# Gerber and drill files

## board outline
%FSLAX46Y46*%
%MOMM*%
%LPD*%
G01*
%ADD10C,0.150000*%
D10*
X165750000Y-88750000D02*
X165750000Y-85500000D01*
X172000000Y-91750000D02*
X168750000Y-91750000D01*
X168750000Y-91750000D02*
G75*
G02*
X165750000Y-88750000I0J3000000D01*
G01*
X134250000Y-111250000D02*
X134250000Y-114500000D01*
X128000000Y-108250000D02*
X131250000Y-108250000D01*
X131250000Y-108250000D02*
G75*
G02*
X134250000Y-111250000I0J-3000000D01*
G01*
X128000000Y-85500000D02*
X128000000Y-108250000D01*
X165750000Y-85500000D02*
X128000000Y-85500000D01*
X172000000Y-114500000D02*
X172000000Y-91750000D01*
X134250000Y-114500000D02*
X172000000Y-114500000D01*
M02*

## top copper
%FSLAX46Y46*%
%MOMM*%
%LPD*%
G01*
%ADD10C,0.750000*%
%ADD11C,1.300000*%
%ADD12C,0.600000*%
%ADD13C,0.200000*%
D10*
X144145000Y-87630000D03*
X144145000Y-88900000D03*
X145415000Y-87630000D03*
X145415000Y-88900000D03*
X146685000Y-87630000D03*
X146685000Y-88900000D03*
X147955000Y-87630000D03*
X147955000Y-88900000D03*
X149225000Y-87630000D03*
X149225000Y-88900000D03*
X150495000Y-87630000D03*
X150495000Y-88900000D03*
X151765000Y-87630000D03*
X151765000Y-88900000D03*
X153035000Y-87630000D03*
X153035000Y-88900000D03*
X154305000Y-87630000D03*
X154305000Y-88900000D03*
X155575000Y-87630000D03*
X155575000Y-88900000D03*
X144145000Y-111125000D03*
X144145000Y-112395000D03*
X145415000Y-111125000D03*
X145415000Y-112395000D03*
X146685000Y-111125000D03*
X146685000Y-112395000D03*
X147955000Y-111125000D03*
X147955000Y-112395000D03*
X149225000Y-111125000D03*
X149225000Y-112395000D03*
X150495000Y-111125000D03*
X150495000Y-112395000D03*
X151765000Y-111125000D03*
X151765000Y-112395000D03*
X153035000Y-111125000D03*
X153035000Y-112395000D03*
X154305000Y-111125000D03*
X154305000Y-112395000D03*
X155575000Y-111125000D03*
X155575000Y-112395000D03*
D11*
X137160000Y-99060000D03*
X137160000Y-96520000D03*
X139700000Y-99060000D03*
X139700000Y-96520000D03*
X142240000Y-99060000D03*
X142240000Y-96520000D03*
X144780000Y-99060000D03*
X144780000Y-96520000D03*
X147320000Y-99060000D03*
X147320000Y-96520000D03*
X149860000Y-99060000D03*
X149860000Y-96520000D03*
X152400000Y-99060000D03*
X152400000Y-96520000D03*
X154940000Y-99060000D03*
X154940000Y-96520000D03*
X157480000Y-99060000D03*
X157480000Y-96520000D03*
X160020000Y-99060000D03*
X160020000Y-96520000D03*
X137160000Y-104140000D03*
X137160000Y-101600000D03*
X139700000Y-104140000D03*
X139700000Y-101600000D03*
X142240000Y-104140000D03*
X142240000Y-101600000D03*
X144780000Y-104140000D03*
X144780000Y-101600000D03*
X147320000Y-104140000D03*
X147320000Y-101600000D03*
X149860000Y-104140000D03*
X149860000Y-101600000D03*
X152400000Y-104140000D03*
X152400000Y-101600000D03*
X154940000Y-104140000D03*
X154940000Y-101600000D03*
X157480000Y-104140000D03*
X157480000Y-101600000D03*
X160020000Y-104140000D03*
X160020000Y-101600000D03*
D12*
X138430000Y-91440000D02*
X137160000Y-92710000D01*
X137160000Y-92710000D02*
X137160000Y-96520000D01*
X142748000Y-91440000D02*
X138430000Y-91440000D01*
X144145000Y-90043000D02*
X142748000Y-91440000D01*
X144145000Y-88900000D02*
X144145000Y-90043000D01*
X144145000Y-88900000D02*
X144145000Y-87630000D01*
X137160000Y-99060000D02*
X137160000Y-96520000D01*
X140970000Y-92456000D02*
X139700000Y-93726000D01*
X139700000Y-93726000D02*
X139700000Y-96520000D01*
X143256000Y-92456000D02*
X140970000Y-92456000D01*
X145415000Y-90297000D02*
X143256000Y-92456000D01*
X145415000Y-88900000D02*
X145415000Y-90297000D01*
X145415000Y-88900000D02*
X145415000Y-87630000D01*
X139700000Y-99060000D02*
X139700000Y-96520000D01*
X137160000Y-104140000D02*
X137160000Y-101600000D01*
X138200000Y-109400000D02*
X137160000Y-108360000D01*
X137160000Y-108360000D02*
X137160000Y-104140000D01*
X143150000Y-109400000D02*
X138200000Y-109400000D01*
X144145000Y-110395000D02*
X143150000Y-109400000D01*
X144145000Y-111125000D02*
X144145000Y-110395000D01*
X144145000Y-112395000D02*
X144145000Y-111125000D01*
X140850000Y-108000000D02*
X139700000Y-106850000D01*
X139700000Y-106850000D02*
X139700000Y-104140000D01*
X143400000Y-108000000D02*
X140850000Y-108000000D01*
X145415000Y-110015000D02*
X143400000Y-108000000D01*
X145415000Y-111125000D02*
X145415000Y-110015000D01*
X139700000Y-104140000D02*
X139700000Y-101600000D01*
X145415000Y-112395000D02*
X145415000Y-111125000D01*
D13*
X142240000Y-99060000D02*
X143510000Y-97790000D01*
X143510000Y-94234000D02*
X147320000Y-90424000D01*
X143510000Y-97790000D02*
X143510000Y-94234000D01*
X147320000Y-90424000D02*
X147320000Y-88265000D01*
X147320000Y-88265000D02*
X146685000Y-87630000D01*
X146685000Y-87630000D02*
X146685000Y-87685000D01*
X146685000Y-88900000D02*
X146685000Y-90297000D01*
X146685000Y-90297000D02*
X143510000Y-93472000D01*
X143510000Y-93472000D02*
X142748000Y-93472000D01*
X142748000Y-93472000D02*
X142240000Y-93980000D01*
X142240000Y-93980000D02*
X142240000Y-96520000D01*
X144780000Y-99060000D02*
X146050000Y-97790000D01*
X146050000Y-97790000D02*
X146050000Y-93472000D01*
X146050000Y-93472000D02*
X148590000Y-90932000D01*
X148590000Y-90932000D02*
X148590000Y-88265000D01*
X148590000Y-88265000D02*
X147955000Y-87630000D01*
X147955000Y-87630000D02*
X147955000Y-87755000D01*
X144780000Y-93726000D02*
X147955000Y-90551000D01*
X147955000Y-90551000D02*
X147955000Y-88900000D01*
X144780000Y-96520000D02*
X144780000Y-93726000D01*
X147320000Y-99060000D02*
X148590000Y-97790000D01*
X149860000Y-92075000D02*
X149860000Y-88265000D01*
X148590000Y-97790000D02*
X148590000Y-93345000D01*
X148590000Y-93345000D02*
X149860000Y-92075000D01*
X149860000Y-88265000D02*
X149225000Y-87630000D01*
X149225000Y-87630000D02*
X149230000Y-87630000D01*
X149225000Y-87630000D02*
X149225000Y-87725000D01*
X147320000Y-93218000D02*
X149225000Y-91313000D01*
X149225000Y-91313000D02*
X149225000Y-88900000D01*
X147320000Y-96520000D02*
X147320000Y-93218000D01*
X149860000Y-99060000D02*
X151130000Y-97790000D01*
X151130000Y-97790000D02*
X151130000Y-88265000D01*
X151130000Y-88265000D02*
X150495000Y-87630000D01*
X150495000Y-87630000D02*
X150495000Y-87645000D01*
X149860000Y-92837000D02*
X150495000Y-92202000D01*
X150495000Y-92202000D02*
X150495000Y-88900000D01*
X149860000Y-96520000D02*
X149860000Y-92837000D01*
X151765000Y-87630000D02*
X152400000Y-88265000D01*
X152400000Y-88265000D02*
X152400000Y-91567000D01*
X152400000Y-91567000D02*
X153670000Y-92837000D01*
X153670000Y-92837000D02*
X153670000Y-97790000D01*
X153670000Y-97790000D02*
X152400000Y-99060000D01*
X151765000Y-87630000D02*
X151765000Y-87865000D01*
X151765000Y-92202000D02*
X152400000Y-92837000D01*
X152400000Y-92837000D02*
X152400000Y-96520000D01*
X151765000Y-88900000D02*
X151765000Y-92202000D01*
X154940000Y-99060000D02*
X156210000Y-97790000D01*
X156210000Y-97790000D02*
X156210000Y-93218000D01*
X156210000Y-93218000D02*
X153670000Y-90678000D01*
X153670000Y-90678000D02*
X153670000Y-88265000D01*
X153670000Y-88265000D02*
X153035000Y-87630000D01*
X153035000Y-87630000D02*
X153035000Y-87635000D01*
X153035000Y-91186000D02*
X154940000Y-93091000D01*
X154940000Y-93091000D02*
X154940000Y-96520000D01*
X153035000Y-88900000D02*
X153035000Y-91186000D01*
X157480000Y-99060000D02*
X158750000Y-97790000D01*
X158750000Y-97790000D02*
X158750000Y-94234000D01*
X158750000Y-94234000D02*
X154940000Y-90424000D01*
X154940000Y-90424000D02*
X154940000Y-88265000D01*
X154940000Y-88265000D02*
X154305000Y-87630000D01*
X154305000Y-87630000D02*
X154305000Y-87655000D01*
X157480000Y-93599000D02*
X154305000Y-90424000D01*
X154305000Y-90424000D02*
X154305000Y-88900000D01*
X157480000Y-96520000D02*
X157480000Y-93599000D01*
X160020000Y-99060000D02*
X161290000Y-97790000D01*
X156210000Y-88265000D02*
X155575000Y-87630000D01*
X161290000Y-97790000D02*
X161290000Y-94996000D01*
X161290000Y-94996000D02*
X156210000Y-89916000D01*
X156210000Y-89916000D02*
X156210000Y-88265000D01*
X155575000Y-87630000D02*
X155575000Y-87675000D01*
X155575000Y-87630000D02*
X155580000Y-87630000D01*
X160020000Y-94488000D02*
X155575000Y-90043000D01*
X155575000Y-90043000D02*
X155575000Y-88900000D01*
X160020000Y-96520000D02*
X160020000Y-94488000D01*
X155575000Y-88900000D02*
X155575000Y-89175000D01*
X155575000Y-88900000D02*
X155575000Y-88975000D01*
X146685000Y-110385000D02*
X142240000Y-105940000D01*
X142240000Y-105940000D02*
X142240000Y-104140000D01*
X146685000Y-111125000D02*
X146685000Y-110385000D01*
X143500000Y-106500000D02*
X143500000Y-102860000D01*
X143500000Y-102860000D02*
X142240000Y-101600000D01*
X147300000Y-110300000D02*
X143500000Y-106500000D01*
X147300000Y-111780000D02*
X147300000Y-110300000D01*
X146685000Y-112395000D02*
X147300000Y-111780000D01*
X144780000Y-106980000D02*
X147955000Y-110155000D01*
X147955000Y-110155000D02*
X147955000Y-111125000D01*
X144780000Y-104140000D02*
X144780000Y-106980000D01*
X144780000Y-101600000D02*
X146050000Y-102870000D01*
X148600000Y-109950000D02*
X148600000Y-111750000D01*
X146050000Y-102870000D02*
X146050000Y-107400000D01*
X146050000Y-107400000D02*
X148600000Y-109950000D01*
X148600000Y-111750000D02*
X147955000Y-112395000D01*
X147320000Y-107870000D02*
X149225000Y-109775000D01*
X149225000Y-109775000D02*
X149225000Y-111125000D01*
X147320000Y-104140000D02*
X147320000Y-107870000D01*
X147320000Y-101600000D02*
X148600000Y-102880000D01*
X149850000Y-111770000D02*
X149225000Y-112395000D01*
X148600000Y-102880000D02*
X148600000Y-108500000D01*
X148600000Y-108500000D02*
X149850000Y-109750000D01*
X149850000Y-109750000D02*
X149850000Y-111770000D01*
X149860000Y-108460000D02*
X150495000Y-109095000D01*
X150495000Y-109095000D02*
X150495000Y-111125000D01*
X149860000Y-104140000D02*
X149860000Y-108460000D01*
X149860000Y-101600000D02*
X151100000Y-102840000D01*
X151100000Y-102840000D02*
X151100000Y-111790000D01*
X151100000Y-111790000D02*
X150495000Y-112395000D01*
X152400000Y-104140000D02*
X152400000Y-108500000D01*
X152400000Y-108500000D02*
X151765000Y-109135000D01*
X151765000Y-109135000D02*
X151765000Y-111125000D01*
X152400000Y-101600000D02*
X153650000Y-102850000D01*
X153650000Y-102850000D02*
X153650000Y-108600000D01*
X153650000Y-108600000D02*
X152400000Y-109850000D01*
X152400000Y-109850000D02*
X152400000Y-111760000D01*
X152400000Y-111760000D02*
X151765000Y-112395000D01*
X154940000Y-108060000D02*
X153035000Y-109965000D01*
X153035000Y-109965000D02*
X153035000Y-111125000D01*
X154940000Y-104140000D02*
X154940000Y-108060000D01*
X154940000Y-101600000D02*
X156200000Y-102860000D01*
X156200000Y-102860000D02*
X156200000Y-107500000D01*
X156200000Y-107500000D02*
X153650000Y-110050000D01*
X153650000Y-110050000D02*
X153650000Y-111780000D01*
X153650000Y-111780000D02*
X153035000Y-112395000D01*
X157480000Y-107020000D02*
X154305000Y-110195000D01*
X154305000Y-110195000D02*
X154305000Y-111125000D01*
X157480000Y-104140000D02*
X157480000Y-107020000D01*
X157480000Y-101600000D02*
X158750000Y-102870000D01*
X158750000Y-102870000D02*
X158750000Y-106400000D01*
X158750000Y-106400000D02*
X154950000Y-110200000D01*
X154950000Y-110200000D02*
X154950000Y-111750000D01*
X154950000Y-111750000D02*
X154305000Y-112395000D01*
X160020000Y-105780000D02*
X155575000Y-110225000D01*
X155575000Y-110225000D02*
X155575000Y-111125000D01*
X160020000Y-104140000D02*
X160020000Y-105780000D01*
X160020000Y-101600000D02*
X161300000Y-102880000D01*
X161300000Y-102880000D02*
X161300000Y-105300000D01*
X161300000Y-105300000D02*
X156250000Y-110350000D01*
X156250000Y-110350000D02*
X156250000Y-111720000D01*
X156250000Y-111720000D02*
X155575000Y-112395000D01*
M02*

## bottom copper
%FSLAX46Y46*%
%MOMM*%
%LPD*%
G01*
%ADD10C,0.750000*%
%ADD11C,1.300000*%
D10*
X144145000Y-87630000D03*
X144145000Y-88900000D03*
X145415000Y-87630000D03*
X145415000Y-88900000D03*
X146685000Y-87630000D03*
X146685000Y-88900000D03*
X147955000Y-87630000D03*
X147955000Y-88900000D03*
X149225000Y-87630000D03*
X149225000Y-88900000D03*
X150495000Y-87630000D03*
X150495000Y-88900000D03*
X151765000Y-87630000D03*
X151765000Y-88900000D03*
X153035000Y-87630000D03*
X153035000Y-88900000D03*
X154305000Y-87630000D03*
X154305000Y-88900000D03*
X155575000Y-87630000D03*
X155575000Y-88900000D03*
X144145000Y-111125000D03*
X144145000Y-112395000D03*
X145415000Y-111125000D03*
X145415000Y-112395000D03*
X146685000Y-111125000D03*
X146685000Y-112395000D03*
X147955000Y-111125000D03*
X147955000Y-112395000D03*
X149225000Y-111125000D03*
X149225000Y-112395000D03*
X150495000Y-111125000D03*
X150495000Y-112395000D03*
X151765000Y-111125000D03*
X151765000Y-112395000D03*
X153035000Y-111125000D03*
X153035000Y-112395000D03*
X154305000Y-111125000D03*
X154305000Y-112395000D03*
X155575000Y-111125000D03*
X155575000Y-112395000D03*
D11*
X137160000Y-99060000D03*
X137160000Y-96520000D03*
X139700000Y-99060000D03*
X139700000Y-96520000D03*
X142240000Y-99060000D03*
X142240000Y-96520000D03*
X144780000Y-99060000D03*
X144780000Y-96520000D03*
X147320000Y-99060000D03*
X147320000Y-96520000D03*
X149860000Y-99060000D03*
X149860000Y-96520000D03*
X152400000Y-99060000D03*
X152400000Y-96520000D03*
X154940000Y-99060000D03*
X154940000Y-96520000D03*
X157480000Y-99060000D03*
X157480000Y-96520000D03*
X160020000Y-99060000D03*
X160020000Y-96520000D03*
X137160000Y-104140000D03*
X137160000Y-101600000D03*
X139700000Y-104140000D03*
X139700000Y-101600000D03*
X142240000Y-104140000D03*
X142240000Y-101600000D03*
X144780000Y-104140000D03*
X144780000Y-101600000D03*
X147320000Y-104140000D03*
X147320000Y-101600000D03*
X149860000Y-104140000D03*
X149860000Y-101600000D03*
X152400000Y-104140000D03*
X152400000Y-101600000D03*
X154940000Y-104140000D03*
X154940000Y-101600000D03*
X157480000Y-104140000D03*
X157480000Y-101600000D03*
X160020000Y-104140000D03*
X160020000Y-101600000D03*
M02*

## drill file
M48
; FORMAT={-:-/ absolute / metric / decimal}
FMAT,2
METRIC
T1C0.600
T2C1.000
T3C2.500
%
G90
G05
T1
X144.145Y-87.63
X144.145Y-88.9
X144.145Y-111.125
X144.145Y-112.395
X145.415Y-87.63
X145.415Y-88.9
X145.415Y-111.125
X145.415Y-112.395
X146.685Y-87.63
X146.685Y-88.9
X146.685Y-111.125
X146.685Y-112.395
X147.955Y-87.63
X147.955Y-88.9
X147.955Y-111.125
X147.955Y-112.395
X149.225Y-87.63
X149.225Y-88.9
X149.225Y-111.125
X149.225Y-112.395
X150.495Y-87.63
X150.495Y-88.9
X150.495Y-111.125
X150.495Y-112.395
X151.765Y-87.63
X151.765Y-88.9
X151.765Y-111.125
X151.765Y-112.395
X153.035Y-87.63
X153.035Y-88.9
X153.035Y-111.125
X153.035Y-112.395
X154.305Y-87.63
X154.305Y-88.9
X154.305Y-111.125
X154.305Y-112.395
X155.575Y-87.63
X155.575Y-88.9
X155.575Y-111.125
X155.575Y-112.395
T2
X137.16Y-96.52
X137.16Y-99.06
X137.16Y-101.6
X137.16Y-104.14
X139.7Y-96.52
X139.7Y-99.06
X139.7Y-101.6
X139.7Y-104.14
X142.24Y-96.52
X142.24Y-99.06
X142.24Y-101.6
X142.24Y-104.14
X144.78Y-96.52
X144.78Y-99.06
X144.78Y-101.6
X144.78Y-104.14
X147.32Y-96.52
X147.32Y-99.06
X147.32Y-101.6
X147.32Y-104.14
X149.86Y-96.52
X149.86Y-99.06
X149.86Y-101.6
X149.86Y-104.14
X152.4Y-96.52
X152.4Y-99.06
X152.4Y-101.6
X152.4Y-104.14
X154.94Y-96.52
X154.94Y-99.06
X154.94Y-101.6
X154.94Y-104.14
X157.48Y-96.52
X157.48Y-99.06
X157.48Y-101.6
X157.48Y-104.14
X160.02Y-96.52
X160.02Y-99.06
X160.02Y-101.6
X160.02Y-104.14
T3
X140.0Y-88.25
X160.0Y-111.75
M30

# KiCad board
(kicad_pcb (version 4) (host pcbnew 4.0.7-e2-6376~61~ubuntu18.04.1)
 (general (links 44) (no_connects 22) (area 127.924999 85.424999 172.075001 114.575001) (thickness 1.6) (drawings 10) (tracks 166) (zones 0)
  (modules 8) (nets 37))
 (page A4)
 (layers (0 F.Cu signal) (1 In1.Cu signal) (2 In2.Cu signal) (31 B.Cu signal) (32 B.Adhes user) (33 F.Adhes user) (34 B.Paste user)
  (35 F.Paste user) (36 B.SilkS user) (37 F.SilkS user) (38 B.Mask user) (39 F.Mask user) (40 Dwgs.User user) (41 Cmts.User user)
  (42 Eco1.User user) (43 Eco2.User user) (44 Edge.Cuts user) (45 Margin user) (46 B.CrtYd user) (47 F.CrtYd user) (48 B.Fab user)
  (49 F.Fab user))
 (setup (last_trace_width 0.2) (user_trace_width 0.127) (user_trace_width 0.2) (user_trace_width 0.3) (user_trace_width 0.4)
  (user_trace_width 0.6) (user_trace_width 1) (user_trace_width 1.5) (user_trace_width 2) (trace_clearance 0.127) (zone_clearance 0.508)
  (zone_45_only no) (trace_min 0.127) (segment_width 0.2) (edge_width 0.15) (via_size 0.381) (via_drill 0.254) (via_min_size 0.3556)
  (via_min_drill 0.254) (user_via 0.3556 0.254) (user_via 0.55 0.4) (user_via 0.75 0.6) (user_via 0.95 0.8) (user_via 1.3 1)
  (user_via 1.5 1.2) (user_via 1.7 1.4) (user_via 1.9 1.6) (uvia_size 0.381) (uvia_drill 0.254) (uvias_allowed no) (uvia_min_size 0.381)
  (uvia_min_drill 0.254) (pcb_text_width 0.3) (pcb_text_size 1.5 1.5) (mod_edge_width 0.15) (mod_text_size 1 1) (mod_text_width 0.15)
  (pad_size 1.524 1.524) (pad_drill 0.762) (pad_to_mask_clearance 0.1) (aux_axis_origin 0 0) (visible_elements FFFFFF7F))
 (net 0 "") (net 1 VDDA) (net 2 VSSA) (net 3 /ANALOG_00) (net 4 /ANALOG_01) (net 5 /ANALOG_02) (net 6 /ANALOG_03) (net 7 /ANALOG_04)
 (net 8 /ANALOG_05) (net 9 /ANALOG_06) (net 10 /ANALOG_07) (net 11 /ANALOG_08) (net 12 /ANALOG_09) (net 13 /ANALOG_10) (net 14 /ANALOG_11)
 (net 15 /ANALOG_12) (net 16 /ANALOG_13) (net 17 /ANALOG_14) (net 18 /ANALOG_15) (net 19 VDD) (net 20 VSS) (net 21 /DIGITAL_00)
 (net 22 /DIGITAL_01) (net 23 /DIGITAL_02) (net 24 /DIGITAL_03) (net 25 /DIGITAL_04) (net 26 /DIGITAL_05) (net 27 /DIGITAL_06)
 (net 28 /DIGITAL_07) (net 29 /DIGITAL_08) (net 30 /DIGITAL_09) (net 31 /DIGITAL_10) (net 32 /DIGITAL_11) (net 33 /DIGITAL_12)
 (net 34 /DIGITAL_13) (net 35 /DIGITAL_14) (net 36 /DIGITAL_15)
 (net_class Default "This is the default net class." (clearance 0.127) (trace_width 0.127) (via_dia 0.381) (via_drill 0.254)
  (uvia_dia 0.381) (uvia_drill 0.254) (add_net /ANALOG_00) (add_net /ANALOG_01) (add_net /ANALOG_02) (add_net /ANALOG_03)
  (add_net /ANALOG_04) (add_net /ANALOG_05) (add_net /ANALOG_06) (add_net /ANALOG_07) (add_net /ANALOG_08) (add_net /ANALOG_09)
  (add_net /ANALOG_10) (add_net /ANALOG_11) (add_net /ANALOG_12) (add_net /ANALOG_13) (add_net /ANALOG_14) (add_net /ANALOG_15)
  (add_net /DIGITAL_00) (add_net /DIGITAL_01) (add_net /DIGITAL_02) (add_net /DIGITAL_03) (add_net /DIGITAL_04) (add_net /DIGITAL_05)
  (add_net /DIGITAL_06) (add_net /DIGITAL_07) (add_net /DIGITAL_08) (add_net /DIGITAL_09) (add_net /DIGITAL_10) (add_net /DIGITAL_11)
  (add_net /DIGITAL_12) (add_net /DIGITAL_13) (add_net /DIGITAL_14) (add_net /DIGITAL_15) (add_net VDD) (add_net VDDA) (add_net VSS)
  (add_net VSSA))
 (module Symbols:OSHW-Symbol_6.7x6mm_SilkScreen (layer F.Cu) (at 165.735 100.33 90)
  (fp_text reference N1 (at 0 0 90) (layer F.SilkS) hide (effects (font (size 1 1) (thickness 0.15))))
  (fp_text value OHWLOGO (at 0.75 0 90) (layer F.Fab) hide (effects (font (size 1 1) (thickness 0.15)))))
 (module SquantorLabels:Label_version (layer F.Cu) (at 170 100 90)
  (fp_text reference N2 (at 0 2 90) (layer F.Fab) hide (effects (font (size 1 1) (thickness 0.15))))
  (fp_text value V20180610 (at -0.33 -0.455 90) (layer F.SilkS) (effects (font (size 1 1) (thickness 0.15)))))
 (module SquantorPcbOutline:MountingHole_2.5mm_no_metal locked (layer F.Cu) (at 140 88.25)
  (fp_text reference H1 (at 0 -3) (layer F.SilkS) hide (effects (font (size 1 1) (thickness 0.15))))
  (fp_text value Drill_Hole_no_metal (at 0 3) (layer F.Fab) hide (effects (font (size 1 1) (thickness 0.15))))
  (pad "" np_thru_hole circle (at 0 0) (size 2.5 2.5) (drill 2.5) (layers *.Cu *.Mask)))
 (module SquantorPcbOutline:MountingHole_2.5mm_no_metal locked (layer F.Cu) (at 160 111.75)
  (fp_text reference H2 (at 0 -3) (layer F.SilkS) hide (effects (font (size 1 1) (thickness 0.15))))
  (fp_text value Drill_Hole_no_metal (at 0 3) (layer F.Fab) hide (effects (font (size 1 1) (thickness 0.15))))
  (pad "" np_thru_hole circle (at 0 0) (size 2.5 2.5) (drill 2.5) (layers *.Cu *.Mask)))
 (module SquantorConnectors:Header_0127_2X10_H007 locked (layer F.Cu) (at 149.86 88.265)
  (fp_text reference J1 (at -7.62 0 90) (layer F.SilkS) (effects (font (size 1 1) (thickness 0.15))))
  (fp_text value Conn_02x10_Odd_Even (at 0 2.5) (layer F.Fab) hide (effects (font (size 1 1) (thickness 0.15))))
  (pad 1 thru_hole circle (at -5.715 -0.635) (size 0.75 0.75) (drill 0.6) (layers *.Cu *.Mask) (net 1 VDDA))
  (pad 2 thru_hole circle (at -5.715 0.635) (size 0.75 0.75) (drill 0.6) (layers *.Cu *.Mask) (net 1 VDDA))
  (pad 3 thru_hole circle (at -4.445 -0.635) (size 0.75 0.75) (drill 0.6) (layers *.Cu *.Mask) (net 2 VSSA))
  (pad 4 thru_hole circle (at -4.445 0.635) (size 0.75 0.75) (drill 0.6) (layers *.Cu *.Mask) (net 2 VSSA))
  (pad 5 thru_hole circle (at -3.175 -0.635) (size 0.75 0.75) (drill 0.6) (layers *.Cu *.Mask) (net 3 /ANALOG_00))
  (pad 6 thru_hole circle (at -3.175 0.635) (size 0.75 0.75) (drill 0.6) (layers *.Cu *.Mask) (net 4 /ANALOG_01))
  (pad 7 thru_hole circle (at -1.905 -0.635) (size 0.75 0.75) (drill 0.6) (layers *.Cu *.Mask) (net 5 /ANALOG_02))
  (pad 8 thru_hole circle (at -1.905 0.635) (size 0.75 0.75) (drill 0.6) (layers *.Cu *.Mask) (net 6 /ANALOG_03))
  (pad 9 thru_hole circle (at -0.635 -0.635) (size 0.75 0.75) (drill 0.6) (layers *.Cu *.Mask) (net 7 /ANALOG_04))
  (pad 10 thru_hole circle (at -0.635 0.635) (size 0.75 0.75) (drill 0.6) (layers *.Cu *.Mask) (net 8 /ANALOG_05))
  (pad 11 thru_hole circle (at 0.635 -0.635) (size 0.75 0.75) (drill 0.6) (layers *.Cu *.Mask) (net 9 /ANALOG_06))
  (pad 12 thru_hole circle (at 0.635 0.635) (size 0.75 0.75) (drill 0.6) (layers *.Cu *.Mask) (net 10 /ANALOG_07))
  (pad 13 thru_hole circle (at 1.905 -0.635) (size 0.75 0.75) (drill 0.6) (layers *.Cu *.Mask) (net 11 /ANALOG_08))
  (pad 14 thru_hole circle (at 1.905 0.635) (size 0.75 0.75) (drill 0.6) (layers *.Cu *.Mask) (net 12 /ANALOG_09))
  (pad 15 thru_hole circle (at 3.175 -0.635) (size 0.75 0.75) (drill 0.6) (layers *.Cu *.Mask) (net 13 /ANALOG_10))
  (pad 16 thru_hole circle (at 3.175 0.635) (size 0.75 0.75) (drill 0.6) (layers *.Cu *.Mask) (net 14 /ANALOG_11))
  (pad 17 thru_hole circle (at 4.445 -0.635) (size 0.75 0.75) (drill 0.6) (layers *.Cu *.Mask) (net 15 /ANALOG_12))
  (pad 18 thru_hole circle (at 4.445 0.635) (size 0.75 0.75) (drill 0.6) (layers *.Cu *.Mask) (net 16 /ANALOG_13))
  (pad 19 thru_hole circle (at 5.715 -0.635) (size 0.75 0.75) (drill 0.6) (layers *.Cu *.Mask) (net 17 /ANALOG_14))
  (pad 20 thru_hole circle (at 5.715 0.635) (size 0.75 0.75) (drill 0.6) (layers *.Cu *.Mask) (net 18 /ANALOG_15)))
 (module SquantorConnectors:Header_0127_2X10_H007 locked (layer F.Cu) (at 149.86 111.76)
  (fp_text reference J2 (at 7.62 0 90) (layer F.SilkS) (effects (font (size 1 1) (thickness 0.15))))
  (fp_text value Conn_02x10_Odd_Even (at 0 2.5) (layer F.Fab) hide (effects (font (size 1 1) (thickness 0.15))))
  (pad 1 thru_hole circle (at -5.715 -0.635) (size 0.75 0.75) (drill 0.6) (layers *.Cu *.Mask) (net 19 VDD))
  (pad 2 thru_hole circle (at -5.715 0.635) (size 0.75 0.75) (drill 0.6) (layers *.Cu *.Mask) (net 19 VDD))
  (pad 3 thru_hole circle (at -4.445 -0.635) (size 0.75 0.75) (drill 0.6) (layers *.Cu *.Mask) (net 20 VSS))
  (pad 4 thru_hole circle (at -4.445 0.635) (size 0.75 0.75) (drill 0.6) (layers *.Cu *.Mask) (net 20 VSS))
  (pad 5 thru_hole circle (at -3.175 -0.635) (size 0.75 0.75) (drill 0.6) (layers *.Cu *.Mask) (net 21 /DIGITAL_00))
  (pad 6 thru_hole circle (at -3.175 0.635) (size 0.75 0.75) (drill 0.6) (layers *.Cu *.Mask) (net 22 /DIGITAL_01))
  (pad 7 thru_hole circle (at -1.905 -0.635) (size 0.75 0.75) (drill 0.6) (layers *.Cu *.Mask) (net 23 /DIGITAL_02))
  (pad 8 thru_hole circle (at -1.905 0.635) (size 0.75 0.75) (drill 0.6) (layers *.Cu *.Mask) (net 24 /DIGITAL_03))
  (pad 9 thru_hole circle (at -0.635 -0.635) (size 0.75 0.75) (drill 0.6) (layers *.Cu *.Mask) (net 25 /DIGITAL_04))
  (pad 10 thru_hole circle (at -0.635 0.635) (size 0.75 0.75) (drill 0.6) (layers *.Cu *.Mask) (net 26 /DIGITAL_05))
  (pad 11 thru_hole circle (at 0.635 -0.635) (size 0.75 0.75) (drill 0.6) (layers *.Cu *.Mask) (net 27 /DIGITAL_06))
  (pad 12 thru_hole circle (at 0.635 0.635) (size 0.75 0.75) (drill 0.6) (layers *.Cu *.Mask) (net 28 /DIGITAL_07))
  (pad 13 thru_hole circle (at 1.905 -0.635) (size 0.75 0.75) (drill 0.6) (layers *.Cu *.Mask) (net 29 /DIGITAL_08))
  (pad 14 thru_hole circle (at 1.905 0.635) (size 0.75 0.75) (drill 0.6) (layers *.Cu *.Mask) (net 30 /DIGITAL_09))
  (pad 15 thru_hole circle (at 3.175 -0.635) (size 0.75 0.75) (drill 0.6) (layers *.Cu *.Mask) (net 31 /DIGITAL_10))
  (pad 16 thru_hole circle (at 3.175 0.635) (size 0.75 0.75) (drill 0.6) (layers *.Cu *.Mask) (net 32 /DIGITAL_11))
  (pad 17 thru_hole circle (at 4.445 -0.635) (size 0.75 0.75) (drill 0.6) (layers *.Cu *.Mask) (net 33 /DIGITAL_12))
  (pad 18 thru_hole circle (at 4.445 0.635) (size 0.75 0.75) (drill 0.6) (layers *.Cu *.Mask) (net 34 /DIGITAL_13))
  (pad 19 thru_hole circle (at 5.715 -0.635) (size 0.75 0.75) (drill 0.6) (layers *.Cu *.Mask) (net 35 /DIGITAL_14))
  (pad 20 thru_hole circle (at 5.715 0.635) (size 0.75 0.75) (drill 0.6) (layers *.Cu *.Mask) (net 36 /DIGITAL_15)))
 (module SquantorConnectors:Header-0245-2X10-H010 (layer F.Cu) (at 148.59 97.79)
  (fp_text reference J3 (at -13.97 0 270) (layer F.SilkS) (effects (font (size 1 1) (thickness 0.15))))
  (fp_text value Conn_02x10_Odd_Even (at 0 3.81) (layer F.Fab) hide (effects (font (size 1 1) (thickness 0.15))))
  (pad 1 thru_hole circle (at -11.43 1.27) (size 1.3 1.3) (drill 1) (layers *.Cu *.Mask) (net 1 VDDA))
  (pad 2 thru_hole circle (at -11.43 -1.27) (size 1.3 1.3) (drill 1) (layers *.Cu *.Mask) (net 1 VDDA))
  (pad 3 thru_hole circle (at -8.89 1.27) (size 1.3 1.3) (drill 1) (layers *.Cu *.Mask) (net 2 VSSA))
  (pad 4 thru_hole circle (at -8.89 -1.27) (size 1.3 1.3) (drill 1) (layers *.Cu *.Mask) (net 2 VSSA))
  (pad 5 thru_hole circle (at -6.35 1.27) (size 1.3 1.3) (drill 1) (layers *.Cu *.Mask) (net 3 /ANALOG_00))
  (pad 6 thru_hole circle (at -6.35 -1.27) (size 1.3 1.3) (drill 1) (layers *.Cu *.Mask) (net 4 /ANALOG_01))
  (pad 7 thru_hole circle (at -3.81 1.27) (size 1.3 1.3) (drill 1) (layers *.Cu *.Mask) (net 5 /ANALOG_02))
  (pad 8 thru_hole circle (at -3.81 -1.27) (size 1.3 1.3) (drill 1) (layers *.Cu *.Mask) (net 6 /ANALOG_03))
  (pad 9 thru_hole circle (at -1.27 1.27) (size 1.3 1.3) (drill 1) (layers *.Cu *.Mask) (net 7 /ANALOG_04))
  (pad 10 thru_hole circle (at -1.27 -1.27) (size 1.3 1.3) (drill 1) (layers *.Cu *.Mask) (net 8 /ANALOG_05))
  (pad 11 thru_hole circle (at 1.27 1.27) (size 1.3 1.3) (drill 1) (layers *.Cu *.Mask) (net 9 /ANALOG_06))
  (pad 12 thru_hole circle (at 1.27 -1.27) (size 1.3 1.3) (drill 1) (layers *.Cu *.Mask) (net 10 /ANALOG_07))
  (pad 13 thru_hole circle (at 3.81 1.27) (size 1.3 1.3) (drill 1) (layers *.Cu *.Mask) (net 11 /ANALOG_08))
  (pad 14 thru_hole circle (at 3.81 -1.27) (size 1.3 1.3) (drill 1) (layers *.Cu *.Mask) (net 12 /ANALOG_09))
  (pad 15 thru_hole circle (at 6.35 1.27) (size 1.3 1.3) (drill 1) (layers *.Cu *.Mask) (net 13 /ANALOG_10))
  (pad 16 thru_hole circle (at 6.35 -1.27) (size 1.3 1.3) (drill 1) (layers *.Cu *.Mask) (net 14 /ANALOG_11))
  (pad 17 thru_hole circle (at 8.89 1.27) (size 1.3 1.3) (drill 1) (layers *.Cu *.Mask) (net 15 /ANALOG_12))
  (pad 18 thru_hole circle (at 8.89 -1.27) (size 1.3 1.3) (drill 1) (layers *.Cu *.Mask) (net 16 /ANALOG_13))
  (pad 19 thru_hole circle (at 11.43 1.27) (size 1.3 1.3) (drill 1) (layers *.Cu *.Mask) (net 17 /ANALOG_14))
  (pad 20 thru_hole circle (at 11.43 -1.27) (size 1.3 1.3) (drill 1) (layers *.Cu *.Mask) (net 18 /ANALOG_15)))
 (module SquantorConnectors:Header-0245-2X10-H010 (layer F.Cu) (at 148.59 102.87)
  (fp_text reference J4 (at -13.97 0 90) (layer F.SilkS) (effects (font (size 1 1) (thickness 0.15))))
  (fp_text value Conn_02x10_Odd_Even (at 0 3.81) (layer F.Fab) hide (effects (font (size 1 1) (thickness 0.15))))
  (pad 1 thru_hole circle (at -11.43 1.27) (size 1.3 1.3) (drill 1) (layers *.Cu *.Mask) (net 19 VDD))
  (pad 2 thru_hole circle (at -11.43 -1.27) (size 1.3 1.3) (drill 1) (layers *.Cu *.Mask) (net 19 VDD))
  (pad 3 thru_hole circle (at -8.89 1.27) (size 1.3 1.3) (drill 1) (layers *.Cu *.Mask) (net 20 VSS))
  (pad 4 thru_hole circle (at -8.89 -1.27) (size 1.3 1.3) (drill 1) (layers *.Cu *.Mask) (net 20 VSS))
  (pad 5 thru_hole circle (at -6.35 1.27) (size 1.3 1.3) (drill 1) (layers *.Cu *.Mask) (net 21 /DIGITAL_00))
  (pad 6 thru_hole circle (at -6.35 -1.27) (size 1.3 1.3) (drill 1) (layers *.Cu *.Mask) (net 22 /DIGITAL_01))
  (pad 7 thru_hole circle (at -3.81 1.27) (size 1.3 1.3) (drill 1) (layers *.Cu *.Mask) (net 23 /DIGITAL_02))
  (pad 8 thru_hole circle (at -3.81 -1.27) (size 1.3 1.3) (drill 1) (layers *.Cu *.Mask) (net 24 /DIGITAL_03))
  (pad 9 thru_hole circle (at -1.27 1.27) (size 1.3 1.3) (drill 1) (layers *.Cu *.Mask) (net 25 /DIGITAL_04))
  (pad 10 thru_hole circle (at -1.27 -1.27) (size 1.3 1.3) (drill 1) (layers *.Cu *.Mask) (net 26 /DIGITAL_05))
  (pad 11 thru_hole circle (at 1.27 1.27) (size 1.3 1.3) (drill 1) (layers *.Cu *.Mask) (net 27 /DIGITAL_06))
  (pad 12 thru_hole circle (at 1.27 -1.27) (size 1.3 1.3) (drill 1) (layers *.Cu *.Mask) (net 28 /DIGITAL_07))
  (pad 13 thru_hole circle (at 3.81 1.27) (size 1.3 1.3) (drill 1) (layers *.Cu *.Mask) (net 29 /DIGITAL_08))
  (pad 14 thru_hole circle (at 3.81 -1.27) (size 1.3 1.3) (drill 1) (layers *.Cu *.Mask) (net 30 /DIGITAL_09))
  (pad 15 thru_hole circle (at 6.35 1.27) (size 1.3 1.3) (drill 1) (layers *.Cu *.Mask) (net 31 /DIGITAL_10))
  (pad 16 thru_hole circle (at 6.35 -1.27) (size 1.3 1.3) (drill 1) (layers *.Cu *.Mask) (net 32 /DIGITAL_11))
  (pad 17 thru_hole circle (at 8.89 1.27) (size 1.3 1.3) (drill 1) (layers *.Cu *.Mask) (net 33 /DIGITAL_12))
  (pad 18 thru_hole circle (at 8.89 -1.27) (size 1.3 1.3) (drill 1) (layers *.Cu *.Mask) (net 34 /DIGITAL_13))
  (pad 19 thru_hole circle (at 11.43 1.27) (size 1.3 1.3) (drill 1) (layers *.Cu *.Mask) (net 35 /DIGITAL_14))
  (pad 20 thru_hole circle (at 11.43 -1.27) (size 1.3 1.3) (drill 1) (layers *.Cu *.Mask) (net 36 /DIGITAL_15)))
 (gr_line (start 165.75 88.75) (end 165.75 85.5) (layer Edge.Cuts) (width 0.15))
 (gr_line (start 172 91.75) (end 168.75 91.75) (layer Edge.Cuts) (width 0.15))
 (gr_arc (start 168.75 88.75) (end 168.75 91.75) (angle 90) (layer Edge.Cuts) (width 0.15))
 (gr_line (start 134.25 111.25) (end 134.25 114.5) (layer Edge.Cuts) (width 0.15))
 (gr_line (start 128 108.25) (end 131.25 108.25) (layer Edge.Cuts) (width 0.15))
 (gr_arc (start 131.25 111.25) (end 131.25 108.25) (angle 90) (layer Edge.Cuts) (width 0.15))
 (gr_line (start 128 85.5) (end 128 108.25) (layer Edge.Cuts) (width 0.15))
 (gr_line (start 165.75 85.5) (end 128 85.5) (layer Edge.Cuts) (width 0.15))
 (gr_line (start 172 114.5) (end 172 91.75) (layer Edge.Cuts) (width 0.15))
 (gr_line (start 134.25 114.5) (end 172 114.5) (layer Edge.Cuts) (width 0.15))
 (segment (start 138.43 91.44) (end 137.16 92.71) (width 0.6) (layer F.Cu) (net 1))
 (segment (start 137.16 92.71) (end 137.16 96.52) (width 0.6) (layer F.Cu) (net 1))
 (segment (start 142.748 91.44) (end 138.43 91.44) (width 0.6) (layer F.Cu) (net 1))
 (segment (start 144.145 90.043) (end 142.748 91.44) (width 0.6) (layer F.Cu) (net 1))
 (segment (start 144.145 88.9) (end 144.145 90.043) (width 0.6) (layer F.Cu) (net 1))
 (segment (start 144.145 88.9) (end 144.145 87.63) (width 0.6) (layer F.Cu) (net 1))
 (segment (start 137.16 99.06) (end 137.16 96.52) (width 0.6) (layer F.Cu) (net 1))
 (segment (start 140.97 92.456) (end 139.7 93.726) (width 0.6) (layer F.Cu) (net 2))
 (segment (start 139.7 93.726) (end 139.7 96.52) (width 0.6) (layer F.Cu) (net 2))
 (segment (start 143.256 92.456) (end 140.97 92.456) (width 0.6) (layer F.Cu) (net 2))
 (segment (start 145.415 90.297) (end 143.256 92.456) (width 0.6) (layer F.Cu) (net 2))
 (segment (start 145.415 88.9) (end 145.415 90.297) (width 0.6) (layer F.Cu) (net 2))
 (segment (start 145.415 88.9) (end 145.415 87.63) (width 0.6) (layer F.Cu) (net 2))
 (segment (start 139.7 99.06) (end 139.7 96.52) (width 0.6) (layer F.Cu) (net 2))
 (segment (start 137.16 104.14) (end 137.16 101.6) (width 0.6) (layer F.Cu) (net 19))
 (segment (start 138.2 109.4) (end 137.16 108.36) (width 0.6) (layer F.Cu) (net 19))
 (segment (start 137.16 108.36) (end 137.16 104.14) (width 0.6) (layer F.Cu) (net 19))
 (segment (start 143.15 109.4) (end 138.2 109.4) (width 0.6) (layer F.Cu) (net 19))
 (segment (start 144.145 110.395) (end 143.15 109.4) (width 0.6) (layer F.Cu) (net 19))
 (segment (start 144.145 111.125) (end 144.145 110.395) (width 0.6) (layer F.Cu) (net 19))
 (segment (start 144.145 112.395) (end 144.145 111.125) (width 0.6) (layer F.Cu) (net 19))
 (segment (start 140.85 108) (end 139.7 106.85) (width 0.6) (layer F.Cu) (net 20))
 (segment (start 139.7 106.85) (end 139.7 104.14) (width 0.6) (layer F.Cu) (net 20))
 (segment (start 143.4 108) (end 140.85 108) (width 0.6) (layer F.Cu) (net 20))
 (segment (start 145.415 110.015) (end 143.4 108) (width 0.6) (layer F.Cu) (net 20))
 (segment (start 145.415 111.125) (end 145.415 110.015) (width 0.6) (layer F.Cu) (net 20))
 (segment (start 139.7 104.14) (end 139.7 101.6) (width 0.6) (layer F.Cu) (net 20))
 (segment (start 145.415 112.395) (end 145.415 111.125) (width 0.6) (layer F.Cu) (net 20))
 (segment (start 142.24 99.06) (end 143.51 97.79) (width 0.2) (layer F.Cu) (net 3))
 (segment (start 143.51 94.234) (end 147.32 90.424) (width 0.2) (layer F.Cu) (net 3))
 (segment (start 143.51 97.79) (end 143.51 94.234) (width 0.2) (layer F.Cu) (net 3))
 (segment (start 147.32 90.424) (end 147.32 88.265) (width 0.2) (layer F.Cu) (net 3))
 (segment (start 147.32 88.265) (end 146.685 87.63) (width 0.2) (layer F.Cu) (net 3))
 (segment (start 146.685 87.63) (end 146.685 87.685) (width 0.2) (layer F.Cu) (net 3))
 (segment (start 146.685 88.9) (end 146.685 90.297) (width 0.2) (layer F.Cu) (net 4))
 (segment (start 146.685 90.297) (end 143.51 93.472) (width 0.2) (layer F.Cu) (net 4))
 (segment (start 143.51 93.472) (end 142.748 93.472) (width 0.2) (layer F.Cu) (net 4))
 (segment (start 142.748 93.472) (end 142.24 93.98) (width 0.2) (layer F.Cu) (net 4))
 (segment (start 142.24 93.98) (end 142.24 96.52) (width 0.2) (layer F.Cu) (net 4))
 (segment (start 144.78 99.06) (end 146.05 97.79) (width 0.2) (layer F.Cu) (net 5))
 (segment (start 146.05 97.79) (end 146.05 93.472) (width 0.2) (layer F.Cu) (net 5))
 (segment (start 146.05 93.472) (end 148.59 90.932) (width 0.2) (layer F.Cu) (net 5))
 (segment (start 148.59 90.932) (end 148.59 88.265) (width 0.2) (layer F.Cu) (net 5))
 (segment (start 148.59 88.265) (end 147.955 87.63) (width 0.2) (layer F.Cu) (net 5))
 (segment (start 147.955 87.63) (end 147.955 87.755) (width 0.2) (layer F.Cu) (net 5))
 (segment (start 144.78 93.726) (end 147.955 90.551) (width 0.2) (layer F.Cu) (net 6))
 (segment (start 147.955 90.551) (end 147.955 88.9) (width 0.2) (layer F.Cu) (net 6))
 (segment (start 144.78 96.52) (end 144.78 93.726) (width 0.2) (layer F.Cu) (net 6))
 (segment (start 147.32 99.06) (end 148.59 97.79) (width 0.2) (layer F.Cu) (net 7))
 (segment (start 149.86 92.075) (end 149.86 88.265) (width 0.2) (layer F.Cu) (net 7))
 (segment (start 148.59 97.79) (end 148.59 93.345) (width 0.2) (layer F.Cu) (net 7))
 (segment (start 148.59 93.345) (end 149.86 92.075) (width 0.2) (layer F.Cu) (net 7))
 (segment (start 149.86 88.265) (end 149.225 87.63) (width 0.2) (layer F.Cu) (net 7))
 (segment (start 149.225 87.63) (end 149.23 87.63) (width 0.2) (layer F.Cu) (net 7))
 (segment (start 149.225 87.63) (end 149.225 87.725) (width 0.2) (layer F.Cu) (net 7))
 (segment (start 147.32 93.218) (end 149.225 91.313) (width 0.2) (layer F.Cu) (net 8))
 (segment (start 149.225 91.313) (end 149.225 88.9) (width 0.2) (layer F.Cu) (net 8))
 (segment (start 147.32 96.52) (end 147.32 93.218) (width 0.2) (layer F.Cu) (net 8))
 (segment (start 149.86 99.06) (end 151.13 97.79) (width 0.2) (layer F.Cu) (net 9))
 (segment (start 151.13 97.79) (end 151.13 88.265) (width 0.2) (layer F.Cu) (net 9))
 (segment (start 151.13 88.265) (end 150.495 87.63) (width 0.2) (layer F.Cu) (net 9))
 (segment (start 150.495 87.63) (end 150.495 87.645) (width 0.2) (layer F.Cu) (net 9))
 (segment (start 149.86 92.837) (end 150.495 92.202) (width 0.2) (layer F.Cu) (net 10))
 (segment (start 150.495 92.202) (end 150.495 88.9) (width 0.2) (layer F.Cu) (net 10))
 (segment (start 149.86 96.52) (end 149.86 92.837) (width 0.2) (layer F.Cu) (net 10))
 (segment (start 151.765 87.63) (end 152.4 88.265) (width 0.2) (layer F.Cu) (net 11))
 (segment (start 152.4 88.265) (end 152.4 91.567) (width 0.2) (layer F.Cu) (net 11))
 (segment (start 152.4 91.567) (end 153.67 92.837) (width 0.2) (layer F.Cu) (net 11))
 (segment (start 153.67 92.837) (end 153.67 97.79) (width 0.2) (layer F.Cu) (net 11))
 (segment (start 153.67 97.79) (end 152.4 99.06) (width 0.2) (layer F.Cu) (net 11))
 (segment (start 151.765 87.63) (end 151.765 87.865) (width 0.2) (layer F.Cu) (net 11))
 (segment (start 151.765 92.202) (end 152.4 92.837) (width 0.2) (layer F.Cu) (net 12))
 (segment (start 152.4 92.837) (end 152.4 96.52) (width 0.2) (layer F.Cu) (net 12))
 (segment (start 151.765 88.9) (end 151.765 92.202) (width 0.2) (layer F.Cu) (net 12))
 (segment (start 154.94 99.06) (end 156.21 97.79) (width 0.2) (layer F.Cu) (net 13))
 (segment (start 156.21 97.79) (end 156.21 93.218) (width 0.2) (layer F.Cu) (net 13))
 (segment (start 156.21 93.218) (end 153.67 90.678) (width 0.2) (layer F.Cu) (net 13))
 (segment (start 153.67 90.678) (end 153.67 88.265) (width 0.2) (layer F.Cu) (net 13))
 (segment (start 153.67 88.265) (end 153.035 87.63) (width 0.2) (layer F.Cu) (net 13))
 (segment (start 153.035 87.63) (end 153.035 87.635) (width 0.2) (layer F.Cu) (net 13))
 (segment (start 153.035 91.186) (end 154.94 93.091) (width 0.2) (layer F.Cu) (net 14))
 (segment (start 154.94 93.091) (end 154.94 96.52) (width 0.2) (layer F.Cu) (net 14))
 (segment (start 153.035 88.9) (end 153.035 91.186) (width 0.2) (layer F.Cu) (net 14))
 (segment (start 157.48 99.06) (end 158.75 97.79) (width 0.2) (layer F.Cu) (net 15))
 (segment (start 158.75 97.79) (end 158.75 94.234) (width 0.2) (layer F.Cu) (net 15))
 (segment (start 158.75 94.234) (end 154.94 90.424) (width 0.2) (layer F.Cu) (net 15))
 (segment (start 154.94 90.424) (end 154.94 88.265) (width 0.2) (layer F.Cu) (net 15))
 (segment (start 154.94 88.265) (end 154.305 87.63) (width 0.2) (layer F.Cu) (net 15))
 (segment (start 154.305 87.63) (end 154.305 87.655) (width 0.2) (layer F.Cu) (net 15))
 (segment (start 157.48 93.599) (end 154.305 90.424) (width 0.2) (layer F.Cu) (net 16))
 (segment (start 154.305 90.424) (end 154.305 88.9) (width 0.2) (layer F.Cu) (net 16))
 (segment (start 157.48 96.52) (end 157.48 93.599) (width 0.2) (layer F.Cu) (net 16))
 (segment (start 160.02 99.06) (end 161.29 97.79) (width 0.2) (layer F.Cu) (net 17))
 (segment (start 156.21 88.265) (end 155.575 87.63) (width 0.2) (layer F.Cu) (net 17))
 (segment (start 161.29 97.79) (end 161.29 94.996) (width 0.2) (layer F.Cu) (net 17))
 (segment (start 161.29 94.996) (end 156.21 89.916) (width 0.2) (layer F.Cu) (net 17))
 (segment (start 156.21 89.916) (end 156.21 88.265) (width 0.2) (layer F.Cu) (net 17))
 (segment (start 155.575 87.63) (end 155.575 87.675) (width 0.2) (layer F.Cu) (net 17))
 (segment (start 155.575 87.63) (end 155.58 87.63) (width 0.2) (layer F.Cu) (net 17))
 (segment (start 160.02 94.488) (end 155.575 90.043) (width 0.2) (layer F.Cu) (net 18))
 (segment (start 155.575 90.043) (end 155.575 88.9) (width 0.2) (layer F.Cu) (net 18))
 (segment (start 160.02 96.52) (end 160.02 94.488) (width 0.2) (layer F.Cu) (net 18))
 (segment (start 155.575 88.9) (end 155.575 89.175) (width 0.2) (layer F.Cu) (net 18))
 (segment (start 155.575 88.9) (end 155.575 88.975) (width 0.2) (layer F.Cu) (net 18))
 (segment (start 146.685 110.385) (end 142.24 105.94) (width 0.2) (layer F.Cu) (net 21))
 (segment (start 142.24 105.94) (end 142.24 104.14) (width 0.2) (layer F.Cu) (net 21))
 (segment (start 146.685 111.125) (end 146.685 110.385) (width 0.2) (layer F.Cu) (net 21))
 (segment (start 143.5 106.5) (end 143.5 102.86) (width 0.2) (layer F.Cu) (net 22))
 (segment (start 143.5 102.86) (end 142.24 101.6) (width 0.2) (layer F.Cu) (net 22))
 (segment (start 147.3 110.3) (end 143.5 106.5) (width 0.2) (layer F.Cu) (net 22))
 (segment (start 147.3 111.78) (end 147.3 110.3) (width 0.2) (layer F.Cu) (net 22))
 (segment (start 146.685 112.395) (end 147.3 111.78) (width 0.2) (layer F.Cu) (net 22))
 (segment (start 144.78 106.98) (end 147.955 110.155) (width 0.2) (layer F.Cu) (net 23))
 (segment (start 147.955 110.155) (end 147.955 111.125) (width 0.2) (layer F.Cu) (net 23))
 (segment (start 144.78 104.14) (end 144.78 106.98) (width 0.2) (layer F.Cu) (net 23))
 (segment (start 144.78 101.6) (end 146.05 102.87) (width 0.2) (layer F.Cu) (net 24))
 (segment (start 148.6 109.95) (end 148.6 111.75) (width 0.2) (layer F.Cu) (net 24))
 (segment (start 146.05 102.87) (end 146.05 107.4) (width 0.2) (layer F.Cu) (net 24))
 (segment (start 146.05 107.4) (end 148.6 109.95) (width 0.2) (layer F.Cu) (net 24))
 (segment (start 148.6 111.75) (end 147.955 112.395) (width 0.2) (layer F.Cu) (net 24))
 (segment (start 147.32 107.87) (end 149.225 109.775) (width 0.2) (layer F.Cu) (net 25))
 (segment (start 149.225 109.775) (end 149.225 111.125) (width 0.2) (layer F.Cu) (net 25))
 (segment (start 147.32 104.14) (end 147.32 107.87) (width 0.2) (layer F.Cu) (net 25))
 (segment (start 147.32 101.6) (end 148.6 102.88) (width 0.2) (layer F.Cu) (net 26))
 (segment (start 149.85 111.77) (end 149.225 112.395) (width 0.2) (layer F.Cu) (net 26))
 (segment (start 148.6 102.88) (end 148.6 108.5) (width 0.2) (layer F.Cu) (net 26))
 (segment (start 148.6 108.5) (end 149.85 109.75) (width 0.2) (layer F.Cu) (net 26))
 (segment (start 149.85 109.75) (end 149.85 111.77) (width 0.2) (layer F.Cu) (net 26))
 (segment (start 149.86 108.46) (end 150.495 109.095) (width 0.2) (layer F.Cu) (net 27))
 (segment (start 150.495 109.095) (end 150.495 111.125) (width 0.2) (layer F.Cu) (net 27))
 (segment (start 149.86 104.14) (end 149.86 108.46) (width 0.2) (layer F.Cu) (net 27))
 (segment (start 149.86 101.6) (end 151.1 102.84) (width 0.2) (layer F.Cu) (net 28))
 (segment (start 151.1 102.84) (end 151.1 111.79) (width 0.2) (layer F.Cu) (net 28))
 (segment (start 151.1 111.79) (end 150.495 112.395) (width 0.2) (layer F.Cu) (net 28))
 (segment (start 152.4 104.14) (end 152.4 108.5) (width 0.2) (layer F.Cu) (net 29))
 (segment (start 152.4 108.5) (end 151.765 109.135) (width 0.2) (layer F.Cu) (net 29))
 (segment (start 151.765 109.135) (end 151.765 111.125) (width 0.2) (layer F.Cu) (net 29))
 (segment (start 152.4 101.6) (end 153.65 102.85) (width 0.2) (layer F.Cu) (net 30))
 (segment (start 153.65 102.85) (end 153.65 108.6) (width 0.2) (layer F.Cu) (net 30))
 (segment (start 153.65 108.6) (end 152.4 109.85) (width 0.2) (layer F.Cu) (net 30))
 (segment (start 152.4 109.85) (end 152.4 111.76) (width 0.2) (layer F.Cu) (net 30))
 (segment (start 152.4 111.76) (end 151.765 112.395) (width 0.2) (layer F.Cu) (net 30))
 (segment (start 154.94 108.06) (end 153.035 109.965) (width 0.2) (layer F.Cu) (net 31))
 (segment (start 153.035 109.965) (end 153.035 111.125) (width 0.2) (layer F.Cu) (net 31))
 (segment (start 154.94 104.14) (end 154.94 108.06) (width 0.2) (layer F.Cu) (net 31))
 (segment (start 154.94 101.6) (end 156.2 102.86) (width 0.2) (layer F.Cu) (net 32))
 (segment (start 156.2 102.86) (end 156.2 107.5) (width 0.2) (layer F.Cu) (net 32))
 (segment (start 156.2 107.5) (end 153.65 110.05) (width 0.2) (layer F.Cu) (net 32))
 (segment (start 153.65 110.05) (end 153.65 111.78) (width 0.2) (layer F.Cu) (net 32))
 (segment (start 153.65 111.78) (end 153.035 112.395) (width 0.2) (layer F.Cu) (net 32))
 (segment (start 157.48 107.02) (end 154.305 110.195) (width 0.2) (layer F.Cu) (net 33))
 (segment (start 154.305 110.195) (end 154.305 111.125) (width 0.2) (layer F.Cu) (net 33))
 (segment (start 157.48 104.14) (end 157.48 107.02) (width 0.2) (layer F.Cu) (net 33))
 (segment (start 157.48 101.6) (end 158.75 102.87) (width 0.2) (layer F.Cu) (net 34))
 (segment (start 158.75 102.87) (end 158.75 106.4) (width 0.2) (layer F.Cu) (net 34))
 (segment (start 158.75 106.4) (end 154.95 110.2) (width 0.2) (layer F.Cu) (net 34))
 (segment (start 154.95 110.2) (end 154.95 111.75) (width 0.2) (layer F.Cu) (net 34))
 (segment (start 154.95 111.75) (end 154.305 112.395) (width 0.2) (layer F.Cu) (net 34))
 (segment (start 160.02 105.78) (end 155.575 110.225) (width 0.2) (layer F.Cu) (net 35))
 (segment (start 155.575 110.225) (end 155.575 111.125) (width 0.2) (layer F.Cu) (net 35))
 (segment (start 160.02 104.14) (end 160.02 105.78) (width 0.2) (layer F.Cu) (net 35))
 (segment (start 160.02 101.6) (end 161.3 102.88) (width 0.2) (layer F.Cu) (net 36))
 (segment (start 161.3 102.88) (end 161.3 105.3) (width 0.2) (layer F.Cu) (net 36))
 (segment (start 161.3 105.3) (end 156.25 110.35) (width 0.2) (layer F.Cu) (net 36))
 (segment (start 156.25 110.35) (end 156.25 111.72) (width 0.2) (layer F.Cu) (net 36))
 (segment (start 156.25 111.72) (end 155.575 112.395) (width 0.2) (layer F.Cu) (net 36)))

